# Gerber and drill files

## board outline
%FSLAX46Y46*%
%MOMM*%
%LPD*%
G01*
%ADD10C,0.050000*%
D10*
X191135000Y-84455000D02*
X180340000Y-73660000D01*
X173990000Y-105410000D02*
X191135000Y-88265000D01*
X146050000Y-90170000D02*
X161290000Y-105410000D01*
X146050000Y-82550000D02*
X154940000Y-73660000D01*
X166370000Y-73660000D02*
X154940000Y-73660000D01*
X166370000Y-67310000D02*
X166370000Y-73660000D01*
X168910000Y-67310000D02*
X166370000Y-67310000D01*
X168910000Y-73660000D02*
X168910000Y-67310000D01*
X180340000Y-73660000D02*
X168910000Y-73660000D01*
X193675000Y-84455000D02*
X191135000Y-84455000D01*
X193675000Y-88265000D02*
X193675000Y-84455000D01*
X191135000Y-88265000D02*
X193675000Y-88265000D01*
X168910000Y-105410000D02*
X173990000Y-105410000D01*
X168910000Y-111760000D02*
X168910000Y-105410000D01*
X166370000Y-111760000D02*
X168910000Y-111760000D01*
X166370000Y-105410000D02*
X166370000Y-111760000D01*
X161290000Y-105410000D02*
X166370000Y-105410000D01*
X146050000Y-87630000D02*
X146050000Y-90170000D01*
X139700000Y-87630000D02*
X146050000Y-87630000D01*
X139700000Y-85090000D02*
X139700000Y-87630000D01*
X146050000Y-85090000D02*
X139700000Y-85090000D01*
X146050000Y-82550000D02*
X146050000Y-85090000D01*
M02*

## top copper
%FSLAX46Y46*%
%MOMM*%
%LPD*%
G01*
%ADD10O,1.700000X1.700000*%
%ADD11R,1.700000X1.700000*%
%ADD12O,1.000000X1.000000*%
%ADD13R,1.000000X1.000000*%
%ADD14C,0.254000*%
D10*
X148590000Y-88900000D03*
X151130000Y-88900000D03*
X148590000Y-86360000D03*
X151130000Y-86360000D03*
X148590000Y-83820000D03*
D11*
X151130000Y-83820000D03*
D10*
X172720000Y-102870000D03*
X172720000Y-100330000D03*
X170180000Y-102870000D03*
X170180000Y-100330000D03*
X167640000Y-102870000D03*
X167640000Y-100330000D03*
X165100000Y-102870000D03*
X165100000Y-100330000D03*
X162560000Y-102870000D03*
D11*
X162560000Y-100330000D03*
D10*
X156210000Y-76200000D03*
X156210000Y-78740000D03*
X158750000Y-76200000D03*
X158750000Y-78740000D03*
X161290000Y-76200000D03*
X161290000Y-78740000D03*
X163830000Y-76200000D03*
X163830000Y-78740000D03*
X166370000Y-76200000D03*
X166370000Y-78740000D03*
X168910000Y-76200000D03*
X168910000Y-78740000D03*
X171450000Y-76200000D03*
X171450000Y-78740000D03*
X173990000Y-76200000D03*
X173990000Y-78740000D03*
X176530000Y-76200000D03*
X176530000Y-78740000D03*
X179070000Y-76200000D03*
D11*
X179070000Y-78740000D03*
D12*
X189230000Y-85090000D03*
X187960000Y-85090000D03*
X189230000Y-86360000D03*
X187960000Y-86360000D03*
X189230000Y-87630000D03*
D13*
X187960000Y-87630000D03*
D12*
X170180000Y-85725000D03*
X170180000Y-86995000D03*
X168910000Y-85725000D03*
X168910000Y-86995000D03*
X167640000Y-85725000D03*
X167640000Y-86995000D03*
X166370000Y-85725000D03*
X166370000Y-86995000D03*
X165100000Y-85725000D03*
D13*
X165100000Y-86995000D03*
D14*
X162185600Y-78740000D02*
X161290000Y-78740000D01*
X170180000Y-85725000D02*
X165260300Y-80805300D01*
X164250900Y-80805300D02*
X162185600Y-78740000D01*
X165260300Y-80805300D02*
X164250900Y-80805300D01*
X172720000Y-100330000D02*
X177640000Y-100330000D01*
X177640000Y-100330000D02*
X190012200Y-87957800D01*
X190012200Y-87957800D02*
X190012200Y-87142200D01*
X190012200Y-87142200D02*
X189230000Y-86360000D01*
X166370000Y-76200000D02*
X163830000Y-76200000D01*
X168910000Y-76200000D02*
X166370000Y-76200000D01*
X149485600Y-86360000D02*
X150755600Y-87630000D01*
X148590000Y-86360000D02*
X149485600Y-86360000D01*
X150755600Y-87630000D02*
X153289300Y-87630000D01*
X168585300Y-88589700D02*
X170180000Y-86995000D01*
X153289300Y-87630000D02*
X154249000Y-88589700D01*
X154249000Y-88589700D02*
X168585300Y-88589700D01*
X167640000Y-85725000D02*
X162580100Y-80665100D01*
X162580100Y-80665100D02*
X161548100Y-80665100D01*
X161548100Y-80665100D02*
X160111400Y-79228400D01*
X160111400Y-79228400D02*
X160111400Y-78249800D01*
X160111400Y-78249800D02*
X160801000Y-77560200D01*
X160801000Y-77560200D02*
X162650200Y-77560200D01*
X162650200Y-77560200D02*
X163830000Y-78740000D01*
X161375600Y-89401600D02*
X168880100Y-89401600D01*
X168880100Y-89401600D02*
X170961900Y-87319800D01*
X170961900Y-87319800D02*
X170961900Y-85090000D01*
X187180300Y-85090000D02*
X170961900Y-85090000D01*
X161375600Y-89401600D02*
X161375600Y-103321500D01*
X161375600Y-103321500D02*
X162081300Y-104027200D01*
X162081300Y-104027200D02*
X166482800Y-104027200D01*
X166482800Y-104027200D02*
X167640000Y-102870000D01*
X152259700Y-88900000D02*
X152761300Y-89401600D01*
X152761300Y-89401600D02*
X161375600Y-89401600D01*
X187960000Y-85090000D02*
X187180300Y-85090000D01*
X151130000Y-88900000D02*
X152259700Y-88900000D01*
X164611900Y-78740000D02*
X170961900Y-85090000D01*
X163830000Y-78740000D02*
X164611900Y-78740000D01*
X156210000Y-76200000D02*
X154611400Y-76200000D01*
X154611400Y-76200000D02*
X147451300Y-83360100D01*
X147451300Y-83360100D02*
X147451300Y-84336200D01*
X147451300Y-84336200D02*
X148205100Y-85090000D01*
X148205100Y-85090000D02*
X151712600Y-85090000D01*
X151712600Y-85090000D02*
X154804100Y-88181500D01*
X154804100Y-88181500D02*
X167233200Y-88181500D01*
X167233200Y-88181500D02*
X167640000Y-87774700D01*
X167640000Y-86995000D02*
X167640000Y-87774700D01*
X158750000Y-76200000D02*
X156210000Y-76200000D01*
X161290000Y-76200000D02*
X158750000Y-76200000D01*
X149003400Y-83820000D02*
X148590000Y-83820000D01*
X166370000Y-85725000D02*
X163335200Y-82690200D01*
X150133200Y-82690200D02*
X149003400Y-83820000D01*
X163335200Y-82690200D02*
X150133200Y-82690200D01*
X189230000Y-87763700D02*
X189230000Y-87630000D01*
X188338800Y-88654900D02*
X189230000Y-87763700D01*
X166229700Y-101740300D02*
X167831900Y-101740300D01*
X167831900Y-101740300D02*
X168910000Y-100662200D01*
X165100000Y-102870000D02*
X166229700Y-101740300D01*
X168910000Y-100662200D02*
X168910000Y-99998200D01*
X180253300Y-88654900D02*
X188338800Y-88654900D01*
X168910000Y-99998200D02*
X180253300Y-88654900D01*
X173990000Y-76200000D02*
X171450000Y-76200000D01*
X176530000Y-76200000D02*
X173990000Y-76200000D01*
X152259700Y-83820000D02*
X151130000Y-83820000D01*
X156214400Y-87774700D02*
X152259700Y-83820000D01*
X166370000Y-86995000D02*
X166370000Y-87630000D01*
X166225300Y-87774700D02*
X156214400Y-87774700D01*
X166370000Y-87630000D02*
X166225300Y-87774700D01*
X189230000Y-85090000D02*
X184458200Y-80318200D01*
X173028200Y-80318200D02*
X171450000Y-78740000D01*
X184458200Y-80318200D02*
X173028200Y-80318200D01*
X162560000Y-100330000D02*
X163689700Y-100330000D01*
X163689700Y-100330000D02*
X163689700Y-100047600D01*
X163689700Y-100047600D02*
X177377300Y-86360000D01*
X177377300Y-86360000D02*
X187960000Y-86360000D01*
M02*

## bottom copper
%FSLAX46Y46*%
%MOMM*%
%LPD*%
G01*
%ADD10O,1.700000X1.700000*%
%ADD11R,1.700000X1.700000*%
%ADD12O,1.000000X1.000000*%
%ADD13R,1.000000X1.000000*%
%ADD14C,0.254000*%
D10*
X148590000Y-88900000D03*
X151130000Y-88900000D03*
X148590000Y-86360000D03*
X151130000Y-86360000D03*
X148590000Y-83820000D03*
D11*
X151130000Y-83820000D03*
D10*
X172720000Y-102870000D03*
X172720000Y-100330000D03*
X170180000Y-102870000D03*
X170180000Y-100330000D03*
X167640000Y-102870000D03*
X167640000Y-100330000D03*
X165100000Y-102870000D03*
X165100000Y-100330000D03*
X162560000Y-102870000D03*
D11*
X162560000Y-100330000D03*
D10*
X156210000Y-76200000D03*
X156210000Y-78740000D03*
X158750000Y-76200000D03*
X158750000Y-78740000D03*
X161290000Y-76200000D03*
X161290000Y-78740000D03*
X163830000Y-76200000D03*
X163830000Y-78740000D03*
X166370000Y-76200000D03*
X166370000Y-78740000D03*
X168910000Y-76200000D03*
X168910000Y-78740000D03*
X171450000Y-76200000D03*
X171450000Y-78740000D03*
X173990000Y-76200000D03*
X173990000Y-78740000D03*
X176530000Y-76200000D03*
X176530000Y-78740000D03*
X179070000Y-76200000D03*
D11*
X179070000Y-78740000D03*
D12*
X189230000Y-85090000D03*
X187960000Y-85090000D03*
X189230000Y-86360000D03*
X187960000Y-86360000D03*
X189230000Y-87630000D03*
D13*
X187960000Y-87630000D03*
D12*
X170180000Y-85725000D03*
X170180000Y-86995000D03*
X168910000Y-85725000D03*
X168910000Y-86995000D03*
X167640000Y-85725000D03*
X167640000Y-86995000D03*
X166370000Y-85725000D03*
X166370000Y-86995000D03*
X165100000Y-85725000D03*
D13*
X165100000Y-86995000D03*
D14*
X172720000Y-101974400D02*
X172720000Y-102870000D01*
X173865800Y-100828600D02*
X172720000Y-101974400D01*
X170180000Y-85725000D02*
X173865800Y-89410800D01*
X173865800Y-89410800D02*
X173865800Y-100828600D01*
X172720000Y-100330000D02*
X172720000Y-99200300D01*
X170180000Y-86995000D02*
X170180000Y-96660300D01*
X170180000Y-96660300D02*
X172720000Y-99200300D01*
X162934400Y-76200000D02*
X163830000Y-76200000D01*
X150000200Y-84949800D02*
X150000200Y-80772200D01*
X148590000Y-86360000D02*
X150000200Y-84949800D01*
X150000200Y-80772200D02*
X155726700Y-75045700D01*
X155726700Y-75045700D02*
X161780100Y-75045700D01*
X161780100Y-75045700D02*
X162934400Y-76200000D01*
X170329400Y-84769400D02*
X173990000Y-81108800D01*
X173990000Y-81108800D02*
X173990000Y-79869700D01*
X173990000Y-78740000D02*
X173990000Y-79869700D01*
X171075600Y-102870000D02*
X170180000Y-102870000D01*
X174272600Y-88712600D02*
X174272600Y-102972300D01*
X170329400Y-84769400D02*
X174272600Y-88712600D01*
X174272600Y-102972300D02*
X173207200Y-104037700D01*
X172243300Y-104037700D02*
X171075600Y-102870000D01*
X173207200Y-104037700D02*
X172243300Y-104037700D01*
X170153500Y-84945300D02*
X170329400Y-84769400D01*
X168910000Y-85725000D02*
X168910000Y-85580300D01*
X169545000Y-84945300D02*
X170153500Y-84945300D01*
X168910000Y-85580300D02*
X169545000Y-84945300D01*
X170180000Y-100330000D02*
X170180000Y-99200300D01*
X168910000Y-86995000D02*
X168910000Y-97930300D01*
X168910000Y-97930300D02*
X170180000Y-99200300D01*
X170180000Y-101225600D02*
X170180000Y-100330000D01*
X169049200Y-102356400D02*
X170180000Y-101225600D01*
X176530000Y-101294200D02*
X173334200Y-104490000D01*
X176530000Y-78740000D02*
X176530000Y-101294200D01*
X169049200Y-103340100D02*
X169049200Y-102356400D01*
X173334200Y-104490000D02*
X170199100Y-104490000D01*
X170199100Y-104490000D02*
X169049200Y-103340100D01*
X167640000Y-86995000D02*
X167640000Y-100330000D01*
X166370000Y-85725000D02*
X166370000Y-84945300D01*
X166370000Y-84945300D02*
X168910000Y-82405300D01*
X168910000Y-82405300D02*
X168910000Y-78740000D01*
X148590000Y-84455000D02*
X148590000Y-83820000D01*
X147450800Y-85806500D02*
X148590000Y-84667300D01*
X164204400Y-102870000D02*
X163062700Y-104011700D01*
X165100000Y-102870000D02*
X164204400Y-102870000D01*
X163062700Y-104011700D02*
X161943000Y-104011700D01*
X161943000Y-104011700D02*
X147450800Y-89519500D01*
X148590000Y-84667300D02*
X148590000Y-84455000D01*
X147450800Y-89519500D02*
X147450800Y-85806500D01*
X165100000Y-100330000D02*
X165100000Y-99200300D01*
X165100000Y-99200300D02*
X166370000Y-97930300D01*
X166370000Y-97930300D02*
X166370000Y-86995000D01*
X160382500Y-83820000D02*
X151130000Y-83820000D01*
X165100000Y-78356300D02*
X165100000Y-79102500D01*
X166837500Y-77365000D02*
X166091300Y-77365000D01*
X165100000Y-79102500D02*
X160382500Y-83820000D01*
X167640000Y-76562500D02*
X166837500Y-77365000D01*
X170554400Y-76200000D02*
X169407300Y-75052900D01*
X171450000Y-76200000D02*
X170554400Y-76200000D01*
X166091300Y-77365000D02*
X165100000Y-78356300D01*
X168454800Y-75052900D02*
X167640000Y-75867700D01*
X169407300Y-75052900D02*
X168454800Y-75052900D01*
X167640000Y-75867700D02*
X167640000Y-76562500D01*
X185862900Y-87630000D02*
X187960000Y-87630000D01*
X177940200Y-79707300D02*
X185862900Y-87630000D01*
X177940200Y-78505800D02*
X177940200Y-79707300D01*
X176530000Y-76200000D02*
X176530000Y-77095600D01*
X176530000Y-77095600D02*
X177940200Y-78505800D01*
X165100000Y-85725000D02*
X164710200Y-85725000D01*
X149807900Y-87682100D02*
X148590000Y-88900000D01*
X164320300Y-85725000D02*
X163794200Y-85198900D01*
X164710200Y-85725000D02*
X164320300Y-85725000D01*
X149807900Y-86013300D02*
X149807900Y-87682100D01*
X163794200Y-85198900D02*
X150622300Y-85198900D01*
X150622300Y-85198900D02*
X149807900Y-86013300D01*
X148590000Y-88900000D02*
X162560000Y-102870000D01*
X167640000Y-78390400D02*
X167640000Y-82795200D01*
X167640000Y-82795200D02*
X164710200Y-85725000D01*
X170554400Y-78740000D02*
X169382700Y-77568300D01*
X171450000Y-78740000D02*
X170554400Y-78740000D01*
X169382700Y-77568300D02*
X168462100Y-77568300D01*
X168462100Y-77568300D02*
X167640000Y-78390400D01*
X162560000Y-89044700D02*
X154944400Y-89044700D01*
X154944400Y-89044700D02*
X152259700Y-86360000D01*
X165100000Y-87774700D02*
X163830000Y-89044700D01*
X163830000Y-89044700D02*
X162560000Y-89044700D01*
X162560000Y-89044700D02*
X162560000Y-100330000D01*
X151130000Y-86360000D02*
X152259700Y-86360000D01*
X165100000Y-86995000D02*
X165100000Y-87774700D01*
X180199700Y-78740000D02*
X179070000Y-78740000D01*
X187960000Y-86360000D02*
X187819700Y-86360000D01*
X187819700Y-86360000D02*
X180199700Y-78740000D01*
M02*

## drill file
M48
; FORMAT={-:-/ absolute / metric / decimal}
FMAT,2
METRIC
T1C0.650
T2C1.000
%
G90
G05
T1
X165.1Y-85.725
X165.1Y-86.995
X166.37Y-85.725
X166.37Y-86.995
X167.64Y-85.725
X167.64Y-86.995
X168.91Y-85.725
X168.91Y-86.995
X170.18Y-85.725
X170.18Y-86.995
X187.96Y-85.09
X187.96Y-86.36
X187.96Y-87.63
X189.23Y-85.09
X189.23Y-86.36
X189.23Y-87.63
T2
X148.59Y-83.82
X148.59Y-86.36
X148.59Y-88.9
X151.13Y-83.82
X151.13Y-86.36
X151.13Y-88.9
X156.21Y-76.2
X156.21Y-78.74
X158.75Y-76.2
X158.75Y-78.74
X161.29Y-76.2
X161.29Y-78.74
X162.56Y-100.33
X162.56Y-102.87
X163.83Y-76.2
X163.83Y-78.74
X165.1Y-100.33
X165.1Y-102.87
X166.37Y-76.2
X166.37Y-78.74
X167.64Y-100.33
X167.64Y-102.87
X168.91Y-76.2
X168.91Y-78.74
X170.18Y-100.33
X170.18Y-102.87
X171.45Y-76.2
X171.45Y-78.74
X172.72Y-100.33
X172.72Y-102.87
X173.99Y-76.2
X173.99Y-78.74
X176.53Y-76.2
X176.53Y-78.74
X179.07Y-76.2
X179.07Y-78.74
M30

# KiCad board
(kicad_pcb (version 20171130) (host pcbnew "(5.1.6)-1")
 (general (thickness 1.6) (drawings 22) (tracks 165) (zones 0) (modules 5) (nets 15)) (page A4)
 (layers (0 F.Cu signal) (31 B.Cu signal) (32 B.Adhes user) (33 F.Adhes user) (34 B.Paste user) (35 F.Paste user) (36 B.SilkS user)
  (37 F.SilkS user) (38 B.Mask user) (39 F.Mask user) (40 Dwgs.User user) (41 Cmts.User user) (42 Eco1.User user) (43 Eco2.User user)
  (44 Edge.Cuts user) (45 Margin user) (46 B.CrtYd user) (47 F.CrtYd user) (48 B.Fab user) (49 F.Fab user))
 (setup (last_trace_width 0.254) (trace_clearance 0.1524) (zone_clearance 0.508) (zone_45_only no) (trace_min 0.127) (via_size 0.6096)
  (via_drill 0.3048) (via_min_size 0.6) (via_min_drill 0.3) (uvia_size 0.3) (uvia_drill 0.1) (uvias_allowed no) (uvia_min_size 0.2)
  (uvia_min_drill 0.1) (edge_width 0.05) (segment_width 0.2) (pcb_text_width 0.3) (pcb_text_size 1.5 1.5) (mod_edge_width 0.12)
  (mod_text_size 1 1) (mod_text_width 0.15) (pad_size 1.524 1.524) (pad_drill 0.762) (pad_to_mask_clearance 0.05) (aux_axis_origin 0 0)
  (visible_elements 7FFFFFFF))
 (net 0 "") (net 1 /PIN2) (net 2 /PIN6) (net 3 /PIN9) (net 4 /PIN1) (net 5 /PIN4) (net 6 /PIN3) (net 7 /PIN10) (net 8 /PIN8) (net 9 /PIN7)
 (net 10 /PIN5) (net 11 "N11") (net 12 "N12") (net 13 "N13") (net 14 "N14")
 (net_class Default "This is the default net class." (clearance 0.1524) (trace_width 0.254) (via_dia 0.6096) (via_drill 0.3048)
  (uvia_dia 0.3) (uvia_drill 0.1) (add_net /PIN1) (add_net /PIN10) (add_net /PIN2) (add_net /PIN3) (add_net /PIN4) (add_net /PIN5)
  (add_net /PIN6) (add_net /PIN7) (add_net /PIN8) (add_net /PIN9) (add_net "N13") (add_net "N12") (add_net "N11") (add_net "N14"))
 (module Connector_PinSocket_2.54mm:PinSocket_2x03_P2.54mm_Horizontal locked (layer F.Cu) (at 151.13 83.82)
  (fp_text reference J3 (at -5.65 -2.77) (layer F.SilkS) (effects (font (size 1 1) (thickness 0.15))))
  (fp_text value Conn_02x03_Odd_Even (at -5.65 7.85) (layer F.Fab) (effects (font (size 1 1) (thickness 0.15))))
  (pad 6 thru_hole oval (at -2.54 5.08) (size 1.7 1.7) (drill 1) (layers *.Cu *.Mask) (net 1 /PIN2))
  (pad 5 thru_hole oval (at 0 5.08) (size 1.7 1.7) (drill 1) (layers *.Cu *.Mask) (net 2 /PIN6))
  (pad 4 thru_hole oval (at -2.54 2.54) (size 1.7 1.7) (drill 1) (layers *.Cu *.Mask) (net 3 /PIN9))
  (pad 3 thru_hole oval (at 0 2.54) (size 1.7 1.7) (drill 1) (layers *.Cu *.Mask) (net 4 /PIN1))
  (pad 2 thru_hole oval (at -2.54 0) (size 1.7 1.7) (drill 1) (layers *.Cu *.Mask) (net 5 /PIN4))
  (pad 1 thru_hole rect (at 0 0) (size 1.7 1.7) (drill 1) (layers *.Cu *.Mask) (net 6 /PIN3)))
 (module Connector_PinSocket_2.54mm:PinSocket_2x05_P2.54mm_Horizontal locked (layer F.Cu) (at 162.56 100.33 90)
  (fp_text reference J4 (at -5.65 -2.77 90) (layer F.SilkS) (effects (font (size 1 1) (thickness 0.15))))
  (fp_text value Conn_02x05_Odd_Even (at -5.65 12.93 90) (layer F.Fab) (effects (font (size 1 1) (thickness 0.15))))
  (pad 10 thru_hole oval (at -2.54 10.16 90) (size 1.7 1.7) (drill 1) (layers *.Cu *.Mask) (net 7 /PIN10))
  (pad 9 thru_hole oval (at 0 10.16 90) (size 1.7 1.7) (drill 1) (layers *.Cu *.Mask) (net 3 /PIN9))
  (pad 8 thru_hole oval (at -2.54 7.62 90) (size 1.7 1.7) (drill 1) (layers *.Cu *.Mask) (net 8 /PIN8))
  (pad 7 thru_hole oval (at 0 7.62 90) (size 1.7 1.7) (drill 1) (layers *.Cu *.Mask) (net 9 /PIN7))
  (pad 6 thru_hole oval (at -2.54 5.08 90) (size 1.7 1.7) (drill 1) (layers *.Cu *.Mask) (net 2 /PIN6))
  (pad 5 thru_hole oval (at 0 5.08 90) (size 1.7 1.7) (drill 1) (layers *.Cu *.Mask) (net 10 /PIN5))
  (pad 4 thru_hole oval (at -2.54 2.54 90) (size 1.7 1.7) (drill 1) (layers *.Cu *.Mask) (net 5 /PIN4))
  (pad 3 thru_hole oval (at 0 2.54 90) (size 1.7 1.7) (drill 1) (layers *.Cu *.Mask) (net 6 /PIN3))
  (pad 2 thru_hole oval (at -2.54 0 90) (size 1.7 1.7) (drill 1) (layers *.Cu *.Mask) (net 1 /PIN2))
  (pad 1 thru_hole rect (at 0 0 90) (size 1.7 1.7) (drill 1) (layers *.Cu *.Mask) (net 4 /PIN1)))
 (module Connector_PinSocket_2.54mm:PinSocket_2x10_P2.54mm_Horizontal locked (layer F.Cu) (at 179.07 78.74 270)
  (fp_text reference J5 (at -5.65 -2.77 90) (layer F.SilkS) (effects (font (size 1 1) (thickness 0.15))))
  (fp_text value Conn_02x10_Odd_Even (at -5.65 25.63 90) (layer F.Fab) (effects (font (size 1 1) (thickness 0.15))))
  (pad 20 thru_hole oval (at -2.54 22.86 270) (size 1.7 1.7) (drill 1) (layers *.Cu *.Mask) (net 10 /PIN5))
  (pad 19 thru_hole oval (at 0 22.86 270) (size 1.7 1.7) (drill 1) (layers *.Cu *.Mask) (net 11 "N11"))
  (pad 18 thru_hole oval (at -2.54 20.32 270) (size 1.7 1.7) (drill 1) (layers *.Cu *.Mask) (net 10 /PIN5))
  (pad 17 thru_hole oval (at 0 20.32 270) (size 1.7 1.7) (drill 1) (layers *.Cu *.Mask) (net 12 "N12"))
  (pad 16 thru_hole oval (at -2.54 17.78 270) (size 1.7 1.7) (drill 1) (layers *.Cu *.Mask) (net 10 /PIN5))
  (pad 15 thru_hole oval (at 0 17.78 270) (size 1.7 1.7) (drill 1) (layers *.Cu *.Mask) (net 7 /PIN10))
  (pad 14 thru_hole oval (at -2.54 15.24 270) (size 1.7 1.7) (drill 1) (layers *.Cu *.Mask) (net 3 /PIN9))
  (pad 13 thru_hole oval (at 0 15.24 270) (size 1.7 1.7) (drill 1) (layers *.Cu *.Mask) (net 2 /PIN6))
  (pad 12 thru_hole oval (at -2.54 12.7 270) (size 1.7 1.7) (drill 1) (layers *.Cu *.Mask) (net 3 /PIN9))
  (pad 11 thru_hole oval (at 0 12.7 270) (size 1.7 1.7) (drill 1) (layers *.Cu *.Mask) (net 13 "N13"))
  (pad 10 thru_hole oval (at -2.54 10.16 270) (size 1.7 1.7) (drill 1) (layers *.Cu *.Mask) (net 3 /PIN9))
  (pad 9 thru_hole oval (at 0 10.16 270) (size 1.7 1.7) (drill 1) (layers *.Cu *.Mask) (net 5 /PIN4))
  (pad 8 thru_hole oval (at -2.54 7.62 270) (size 1.7 1.7) (drill 1) (layers *.Cu *.Mask) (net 6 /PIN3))
  (pad 7 thru_hole oval (at 0 7.62 270) (size 1.7 1.7) (drill 1) (layers *.Cu *.Mask) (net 1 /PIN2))
  (pad 6 thru_hole oval (at -2.54 5.08 270) (size 1.7 1.7) (drill 1) (layers *.Cu *.Mask) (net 6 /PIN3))
  (pad 5 thru_hole oval (at 0 5.08 270) (size 1.7 1.7) (drill 1) (layers *.Cu *.Mask) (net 8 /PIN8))
  (pad 4 thru_hole oval (at -2.54 2.54 270) (size 1.7 1.7) (drill 1) (layers *.Cu *.Mask) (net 6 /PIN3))
  (pad 3 thru_hole oval (at 0 2.54 270) (size 1.7 1.7) (drill 1) (layers *.Cu *.Mask) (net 9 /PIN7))
  (pad 2 thru_hole oval (at -2.54 0 270) (size 1.7 1.7) (drill 1) (layers *.Cu *.Mask) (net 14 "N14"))
  (pad 1 thru_hole rect (at 0 0 270) (size 1.7 1.7) (drill 1) (layers *.Cu *.Mask) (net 4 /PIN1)))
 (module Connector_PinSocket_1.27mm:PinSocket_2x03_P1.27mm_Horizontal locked (layer F.Cu) (at 187.96 87.63 180)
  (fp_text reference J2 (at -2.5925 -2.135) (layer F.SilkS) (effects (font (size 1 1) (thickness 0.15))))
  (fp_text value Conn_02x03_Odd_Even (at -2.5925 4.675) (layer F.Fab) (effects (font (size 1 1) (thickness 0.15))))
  (pad 6 thru_hole oval (at -1.27 2.54 180) (size 1 1) (drill 0.65) (layers *.Cu *.Mask) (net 1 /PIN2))
  (pad 5 thru_hole oval (at 0 2.54 180) (size 1 1) (drill 0.65) (layers *.Cu *.Mask) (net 2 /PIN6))
  (pad 4 thru_hole oval (at -1.27 1.27 180) (size 1 1) (drill 0.65) (layers *.Cu *.Mask) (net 3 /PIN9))
  (pad 3 thru_hole oval (at 0 1.27 180) (size 1 1) (drill 0.65) (layers *.Cu *.Mask) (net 4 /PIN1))
  (pad 2 thru_hole oval (at -1.27 0 180) (size 1 1) (drill 0.65) (layers *.Cu *.Mask) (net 5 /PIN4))
  (pad 1 thru_hole rect (at 0 0 180) (size 1 1) (drill 0.65) (layers *.Cu *.Mask) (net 6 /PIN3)))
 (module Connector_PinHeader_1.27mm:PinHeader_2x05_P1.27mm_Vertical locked (layer F.Cu) (at 165.1 86.995 90)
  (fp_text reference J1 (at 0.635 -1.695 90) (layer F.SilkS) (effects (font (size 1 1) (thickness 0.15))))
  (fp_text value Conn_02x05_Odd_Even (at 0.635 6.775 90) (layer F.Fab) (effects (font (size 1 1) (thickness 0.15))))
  (pad 10 thru_hole oval (at 1.27 5.08 90) (size 1 1) (drill 0.65) (layers *.Cu *.Mask) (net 7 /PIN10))
  (pad 9 thru_hole oval (at 0 5.08 90) (size 1 1) (drill 0.65) (layers *.Cu *.Mask) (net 3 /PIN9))
  (pad 8 thru_hole oval (at 1.27 3.81 90) (size 1 1) (drill 0.65) (layers *.Cu *.Mask) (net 8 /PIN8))
  (pad 7 thru_hole oval (at 0 3.81 90) (size 1 1) (drill 0.65) (layers *.Cu *.Mask) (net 9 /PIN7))
  (pad 6 thru_hole oval (at 1.27 2.54 90) (size 1 1) (drill 0.65) (layers *.Cu *.Mask) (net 2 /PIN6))
  (pad 5 thru_hole oval (at 0 2.54 90) (size 1 1) (drill 0.65) (layers *.Cu *.Mask) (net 10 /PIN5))
  (pad 4 thru_hole oval (at 1.27 1.27 90) (size 1 1) (drill 0.65) (layers *.Cu *.Mask) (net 5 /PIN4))
  (pad 3 thru_hole oval (at 0 1.27 90) (size 1 1) (drill 0.65) (layers *.Cu *.Mask) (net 6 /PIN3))
  (pad 2 thru_hole oval (at 1.27 0 90) (size 1 1) (drill 0.65) (layers *.Cu *.Mask) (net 1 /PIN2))
  (pad 1 thru_hole rect (at 0 0 90) (size 1 1) (drill 0.65) (layers *.Cu *.Mask) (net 4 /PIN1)))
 (gr_line (start 191.135 84.455) (end 180.34 73.66) (layer Edge.Cuts) (width 0.05))
 (gr_line (start 173.99 105.41) (end 191.135 88.265) (layer Edge.Cuts) (width 0.05))
 (gr_line (start 146.05 90.17) (end 161.29 105.41) (layer Edge.Cuts) (width 0.05))
 (gr_line (start 146.05 82.55) (end 154.94 73.66) (layer Edge.Cuts) (width 0.05))
 (gr_line (start 166.37 73.66) (end 154.94 73.66) (layer Edge.Cuts) (width 0.05))
 (gr_line (start 166.37 67.31) (end 166.37 73.66) (layer Edge.Cuts) (width 0.05))
 (gr_line (start 168.91 67.31) (end 166.37 67.31) (layer Edge.Cuts) (width 0.05))
 (gr_line (start 168.91 73.66) (end 168.91 67.31) (layer Edge.Cuts) (width 0.05))
 (gr_line (start 180.34 73.66) (end 168.91 73.66) (layer Edge.Cuts) (width 0.05))
 (gr_line (start 193.675 84.455) (end 191.135 84.455) (layer Edge.Cuts) (width 0.05))
 (gr_line (start 193.675 88.265) (end 193.675 84.455) (layer Edge.Cuts) (width 0.05))
 (gr_line (start 191.135 88.265) (end 193.675 88.265) (layer Edge.Cuts) (width 0.05))
 (gr_line (start 168.91 105.41) (end 173.99 105.41) (layer Edge.Cuts) (width 0.05))
 (gr_line (start 168.91 111.76) (end 168.91 105.41) (layer Edge.Cuts) (width 0.05))
 (gr_line (start 166.37 111.76) (end 168.91 111.76) (layer Edge.Cuts) (width 0.05))
 (gr_line (start 166.37 105.41) (end 166.37 111.76) (layer Edge.Cuts) (width 0.05))
 (gr_line (start 161.29 105.41) (end 166.37 105.41) (layer Edge.Cuts) (width 0.05))
 (gr_line (start 146.05 87.63) (end 146.05 90.17) (layer Edge.Cuts) (width 0.05))
 (gr_line (start 139.7 87.63) (end 146.05 87.63) (layer Edge.Cuts) (width 0.05))
 (gr_line (start 139.7 85.09) (end 139.7 87.63) (layer Edge.Cuts) (width 0.05))
 (gr_line (start 146.05 85.09) (end 139.7 85.09) (layer Edge.Cuts) (width 0.05))
 (gr_line (start 146.05 82.55) (end 146.05 85.09) (layer Edge.Cuts) (width 0.05))
 (segment (start 162.1856 78.74) (end 161.29 78.74) (width 0.254) (layer F.Cu) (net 7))
 (segment (start 170.18 85.725) (end 165.2603 80.8053) (width 0.254) (layer F.Cu) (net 7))
 (segment (start 164.2509 80.8053) (end 162.1856 78.74) (width 0.254) (layer F.Cu) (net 7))
 (segment (start 165.2603 80.8053) (end 164.2509 80.8053) (width 0.254) (layer F.Cu) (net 7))
 (segment (start 172.72 101.9744) (end 172.72 102.87) (width 0.254) (layer B.Cu) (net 7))
 (segment (start 173.8658 100.8286) (end 172.72 101.9744) (width 0.254) (layer B.Cu) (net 7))
 (segment (start 170.18 85.725) (end 173.8658 89.4108) (width 0.254) (layer B.Cu) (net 7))
 (segment (start 173.8658 89.4108) (end 173.8658 100.8286) (width 0.254) (layer B.Cu) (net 7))
 (segment (start 172.72 100.33) (end 172.72 99.2003) (width 0.254) (layer B.Cu) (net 3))
 (segment (start 170.18 86.995) (end 170.18 96.6603) (width 0.254) (layer B.Cu) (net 3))
 (segment (start 170.18 96.6603) (end 172.72 99.2003) (width 0.254) (layer B.Cu) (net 3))
 (segment (start 172.72 100.33) (end 177.64 100.33) (width 0.254) (layer F.Cu) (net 3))
 (segment (start 177.64 100.33) (end 190.0122 87.9578) (width 0.254) (layer F.Cu) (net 3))
 (segment (start 190.0122 87.9578) (end 190.0122 87.1422) (width 0.254) (layer F.Cu) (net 3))
 (segment (start 190.0122 87.1422) (end 189.23 86.36) (width 0.254) (layer F.Cu) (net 3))
 (segment (start 166.37 76.2) (end 163.83 76.2) (width 0.254) (layer F.Cu) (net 3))
 (segment (start 168.91 76.2) (end 166.37 76.2) (width 0.254) (layer F.Cu) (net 3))
 (segment (start 149.4856 86.36) (end 150.7556 87.63) (width 0.254) (layer F.Cu) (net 3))
 (segment (start 148.59 86.36) (end 149.4856 86.36) (width 0.254) (layer F.Cu) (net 3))
 (segment (start 150.7556 87.63) (end 153.2893 87.63) (width 0.254) (layer F.Cu) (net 3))
 (segment (start 168.5853 88.5897) (end 170.18 86.995) (width 0.254) (layer F.Cu) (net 3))
 (segment (start 153.2893 87.63) (end 154.249 88.5897) (width 0.254) (layer F.Cu) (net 3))
 (segment (start 154.249 88.5897) (end 168.5853 88.5897) (width 0.254) (layer F.Cu) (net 3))
 (segment (start 162.9344 76.2) (end 163.83 76.2) (width 0.254) (layer B.Cu) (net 3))
 (segment (start 150.0002 84.9498) (end 150.0002 80.7722) (width 0.254) (layer B.Cu) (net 3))
 (segment (start 148.59 86.36) (end 150.0002 84.9498) (width 0.254) (layer B.Cu) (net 3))
 (segment (start 150.0002 80.7722) (end 155.7267 75.0457) (width 0.254) (layer B.Cu) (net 3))
 (segment (start 155.7267 75.0457) (end 161.7801 75.0457) (width 0.254) (layer B.Cu) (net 3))
 (segment (start 161.7801 75.0457) (end 162.9344 76.2) (width 0.254) (layer B.Cu) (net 3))
 (segment (start 170.3294 84.7694) (end 173.99 81.1088) (width 0.254) (layer B.Cu) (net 8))
 (segment (start 173.99 81.1088) (end 173.99 79.8697) (width 0.254) (layer B.Cu) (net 8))
 (segment (start 173.99 78.74) (end 173.99 79.8697) (width 0.254) (layer B.Cu) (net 8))
 (segment (start 171.0756 102.87) (end 170.18 102.87) (width 0.254) (layer B.Cu) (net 8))
 (segment (start 174.2726 88.7126) (end 174.2726 102.9723) (width 0.254) (layer B.Cu) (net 8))
 (segment (start 170.3294 84.7694) (end 174.2726 88.7126) (width 0.254) (layer B.Cu) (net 8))
 (segment (start 174.2726 102.9723) (end 173.2072 104.0377) (width 0.254) (layer B.Cu) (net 8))
 (segment (start 172.2433 104.0377) (end 171.0756 102.87) (width 0.254) (layer B.Cu) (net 8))
 (segment (start 173.2072 104.0377) (end 172.2433 104.0377) (width 0.254) (layer B.Cu) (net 8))
 (segment (start 170.1535 84.9453) (end 170.3294 84.7694) (width 0.254) (layer B.Cu) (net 8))
 (segment (start 168.91 85.725) (end 168.91 85.5803) (width 0.254) (layer B.Cu) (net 8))
 (segment (start 169.545 84.9453) (end 170.1535 84.9453) (width 0.254) (layer B.Cu) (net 8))
 (segment (start 168.91 85.5803) (end 169.545 84.9453) (width 0.254) (layer B.Cu) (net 8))
 (segment (start 170.18 100.33) (end 170.18 99.2003) (width 0.254) (layer B.Cu) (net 9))
 (segment (start 168.91 86.995) (end 168.91 97.9303) (width 0.254) (layer B.Cu) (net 9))
 (segment (start 168.91 97.9303) (end 170.18 99.2003) (width 0.254) (layer B.Cu) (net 9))
 (segment (start 170.18 101.2256) (end 170.18 100.33) (width 0.254) (layer B.Cu) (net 9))
 (segment (start 169.0492 102.3564) (end 170.18 101.2256) (width 0.254) (layer B.Cu) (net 9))
 (segment (start 176.53 101.2942) (end 173.3342 104.49) (width 0.254) (layer B.Cu) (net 9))
 (segment (start 176.53 78.74) (end 176.53 101.2942) (width 0.254) (layer B.Cu) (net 9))
 (segment (start 169.0492 103.3401) (end 169.0492 102.3564) (width 0.254) (layer B.Cu) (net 9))
 (segment (start 173.3342 104.49) (end 170.1991 104.49) (width 0.254) (layer B.Cu) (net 9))
 (segment (start 170.1991 104.49) (end 169.0492 103.3401) (width 0.254) (layer B.Cu) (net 9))
 (segment (start 167.64 85.725) (end 162.5801 80.6651) (width 0.254) (layer F.Cu) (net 2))
 (segment (start 162.5801 80.6651) (end 161.5481 80.6651) (width 0.254) (layer F.Cu) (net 2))
 (segment (start 161.5481 80.6651) (end 160.1114 79.2284) (width 0.254) (layer F.Cu) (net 2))
 (segment (start 160.1114 79.2284) (end 160.1114 78.2498) (width 0.254) (layer F.Cu) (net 2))
 (segment (start 160.1114 78.2498) (end 160.801 77.5602) (width 0.254) (layer F.Cu) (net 2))
 (segment (start 160.801 77.5602) (end 162.6502 77.5602) (width 0.254) (layer F.Cu) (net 2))
 (segment (start 162.6502 77.5602) (end 163.83 78.74) (width 0.254) (layer F.Cu) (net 2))
 (segment (start 161.3756 89.4016) (end 168.8801 89.4016) (width 0.254) (layer F.Cu) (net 2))
 (segment (start 168.8801 89.4016) (end 170.9619 87.3198) (width 0.254) (layer F.Cu) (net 2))
 (segment (start 170.9619 87.3198) (end 170.9619 85.09) (width 0.254) (layer F.Cu) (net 2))
 (segment (start 187.1803 85.09) (end 170.9619 85.09) (width 0.254) (layer F.Cu) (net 2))
 (segment (start 161.3756 89.4016) (end 161.3756 103.3215) (width 0.254) (layer F.Cu) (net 2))
 (segment (start 161.3756 103.3215) (end 162.0813 104.0272) (width 0.254) (layer F.Cu) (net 2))
 (segment (start 162.0813 104.0272) (end 166.4828 104.0272) (width 0.254) (layer F.Cu) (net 2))
 (segment (start 166.4828 104.0272) (end 167.64 102.87) (width 0.254) (layer F.Cu) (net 2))
 (segment (start 152.2597 88.9) (end 152.7613 89.4016) (width 0.254) (layer F.Cu) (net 2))
 (segment (start 152.7613 89.4016) (end 161.3756 89.4016) (width 0.254) (layer F.Cu) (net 2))
 (segment (start 187.96 85.09) (end 187.1803 85.09) (width 0.254) (layer F.Cu) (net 2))
 (segment (start 151.13 88.9) (end 152.2597 88.9) (width 0.254) (layer F.Cu) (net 2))
 (segment (start 164.6119 78.74) (end 170.9619 85.09) (width 0.254) (layer F.Cu) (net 2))
 (segment (start 163.83 78.74) (end 164.6119 78.74) (width 0.254) (layer F.Cu) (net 2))
 (segment (start 156.21 76.2) (end 154.6114 76.2) (width 0.254) (layer F.Cu) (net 10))
 (segment (start 154.6114 76.2) (end 147.4513 83.3601) (width 0.254) (layer F.Cu) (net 10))
 (segment (start 147.4513 83.3601) (end 147.4513 84.3362) (width 0.254) (layer F.Cu) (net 10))
 (segment (start 147.4513 84.3362) (end 148.2051 85.09) (width 0.254) (layer F.Cu) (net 10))
 (segment (start 148.2051 85.09) (end 151.7126 85.09) (width 0.254) (layer F.Cu) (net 10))
 (segment (start 151.7126 85.09) (end 154.8041 88.1815) (width 0.254) (layer F.Cu) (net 10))
 (segment (start 154.8041 88.1815) (end 167.2332 88.1815) (width 0.254) (layer F.Cu) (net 10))
 (segment (start 167.2332 88.1815) (end 167.64 87.7747) (width 0.254) (layer F.Cu) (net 10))
 (segment (start 167.64 86.995) (end 167.64 87.7747) (width 0.254) (layer F.Cu) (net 10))
 (segment (start 167.64 86.995) (end 167.64 100.33) (width 0.254) (layer B.Cu) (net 10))
 (segment (start 158.75 76.2) (end 156.21 76.2) (width 0.254) (layer F.Cu) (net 10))
 (segment (start 161.29 76.2) (end 158.75 76.2) (width 0.254) (layer F.Cu) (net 10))
 (segment (start 166.37 85.725) (end 166.37 84.9453) (width 0.254) (layer B.Cu) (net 5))
 (segment (start 166.37 84.9453) (end 168.91 82.4053) (width 0.254) (layer B.Cu) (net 5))
 (segment (start 168.91 82.4053) (end 168.91 78.74) (width 0.254) (layer B.Cu) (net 5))
 (segment (start 149.0034 83.82) (end 148.59 83.82) (width 0.254) (layer F.Cu) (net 5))
 (segment (start 166.37 85.725) (end 163.3352 82.6902) (width 0.254) (layer F.Cu) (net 5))
 (segment (start 150.1332 82.6902) (end 149.0034 83.82) (width 0.254) (layer F.Cu) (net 5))
 (segment (start 163.3352 82.6902) (end 150.1332 82.6902) (width 0.254) (layer F.Cu) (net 5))
 (segment (start 148.59 84.455) (end 148.59 83.82) (width 0.254) (layer B.Cu) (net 5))
 (segment (start 147.4508 85.8065) (end 148.59 84.6673) (width 0.254) (layer B.Cu) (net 5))
 (segment (start 164.2044 102.87) (end 163.0627 104.0117) (width 0.254) (layer B.Cu) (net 5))
 (segment (start 165.1 102.87) (end 164.2044 102.87) (width 0.254) (layer B.Cu) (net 5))
 (segment (start 163.0627 104.0117) (end 161.943 104.0117) (width 0.254) (layer B.Cu) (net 5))
 (segment (start 161.943 104.0117) (end 147.4508 89.5195) (width 0.254) (layer B.Cu) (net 5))
 (segment (start 148.59 84.6673) (end 148.59 84.455) (width 0.254) (layer B.Cu) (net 5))
 (segment (start 147.4508 89.5195) (end 147.4508 85.8065) (width 0.254) (layer B.Cu) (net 5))
 (segment (start 189.23 87.7637) (end 189.23 87.63) (width 0.254) (layer F.Cu) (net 5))
 (segment (start 188.3388 88.6549) (end 189.23 87.7637) (width 0.254) (layer F.Cu) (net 5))
 (segment (start 166.2297 101.7403) (end 167.8319 101.7403) (width 0.254) (layer F.Cu) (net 5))
 (segment (start 167.8319 101.7403) (end 168.91 100.6622) (width 0.254) (layer F.Cu) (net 5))
 (segment (start 165.1 102.87) (end 166.2297 101.7403) (width 0.254) (layer F.Cu) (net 5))
 (segment (start 168.91 100.6622) (end 168.91 99.9982) (width 0.254) (layer F.Cu) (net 5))
 (segment (start 180.2533 88.6549) (end 188.3388 88.6549) (width 0.254) (layer F.Cu) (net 5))
 (segment (start 168.91 99.9982) (end 180.2533 88.6549) (width 0.254) (layer F.Cu) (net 5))
 (segment (start 173.99 76.2) (end 171.45 76.2) (width 0.254) (layer F.Cu) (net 6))
 (segment (start 165.1 100.33) (end 165.1 99.2003) (width 0.254) (layer B.Cu) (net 6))
 (segment (start 165.1 99.2003) (end 166.37 97.9303) (width 0.254) (layer B.Cu) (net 6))
 (segment (start 166.37 97.9303) (end 166.37 86.995) (width 0.254) (layer B.Cu) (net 6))
 (segment (start 176.53 76.2) (end 173.99 76.2) (width 0.254) (layer F.Cu) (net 6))
 (segment (start 160.3825 83.82) (end 151.13 83.82) (width 0.254) (layer B.Cu) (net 6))
 (segment (start 165.1 78.3563) (end 165.1 79.1025) (width 0.254) (layer B.Cu) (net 6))
 (segment (start 166.8375 77.365) (end 166.0913 77.365) (width 0.254) (layer B.Cu) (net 6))
 (segment (start 165.1 79.1025) (end 160.3825 83.82) (width 0.254) (layer B.Cu) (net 6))
 (segment (start 167.64 76.5625) (end 166.8375 77.365) (width 0.254) (layer B.Cu) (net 6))
 (segment (start 170.5544 76.2) (end 169.4073 75.0529) (width 0.254) (layer B.Cu) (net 6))
 (segment (start 171.45 76.2) (end 170.5544 76.2) (width 0.254) (layer B.Cu) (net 6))
 (segment (start 166.0913 77.365) (end 165.1 78.3563) (width 0.254) (layer B.Cu) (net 6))
 (segment (start 168.4548 75.0529) (end 167.64 75.8677) (width 0.254) (layer B.Cu) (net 6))
 (segment (start 169.4073 75.0529) (end 168.4548 75.0529) (width 0.254) (layer B.Cu) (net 6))
 (segment (start 167.64 75.8677) (end 167.64 76.5625) (width 0.254) (layer B.Cu) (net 6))
 (segment (start 185.8629 87.63) (end 187.96 87.63) (width 0.254) (layer B.Cu) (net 6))
 (segment (start 177.9402 79.7073) (end 185.8629 87.63) (width 0.254) (layer B.Cu) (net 6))
 (segment (start 177.9402 78.5058) (end 177.9402 79.7073) (width 0.254) (layer B.Cu) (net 6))
 (segment (start 176.53 76.2) (end 176.53 77.0956) (width 0.254) (layer B.Cu) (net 6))
 (segment (start 176.53 77.0956) (end 177.9402 78.5058) (width 0.254) (layer B.Cu) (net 6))
 (segment (start 152.2597 83.82) (end 151.13 83.82) (width 0.254) (layer F.Cu) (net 6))
 (segment (start 156.2144 87.7747) (end 152.2597 83.82) (width 0.254) (layer F.Cu) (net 6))
 (segment (start 166.37 86.995) (end 166.37 87.63) (width 0.254) (layer F.Cu) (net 6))
 (segment (start 166.2253 87.7747) (end 156.2144 87.7747) (width 0.254) (layer F.Cu) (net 6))
 (segment (start 166.37 87.63) (end 166.2253 87.7747) (width 0.254) (layer F.Cu) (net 6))
 (segment (start 165.1 85.725) (end 164.7102 85.725) (width 0.254) (layer B.Cu) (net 1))
 (segment (start 149.8079 87.6821) (end 148.59 88.9) (width 0.254) (layer B.Cu) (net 1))
 (segment (start 164.3203 85.725) (end 163.7942 85.1989) (width 0.254) (layer B.Cu) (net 1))
 (segment (start 164.7102 85.725) (end 164.3203 85.725) (width 0.254) (layer B.Cu) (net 1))
 (segment (start 149.8079 86.0133) (end 149.8079 87.6821) (width 0.254) (layer B.Cu) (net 1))
 (segment (start 163.7942 85.1989) (end 150.6223 85.1989) (width 0.254) (layer B.Cu) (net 1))
 (segment (start 150.6223 85.1989) (end 149.8079 86.0133) (width 0.254) (layer B.Cu) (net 1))
 (segment (start 148.59 88.9) (end 162.56 102.87) (width 0.254) (layer B.Cu) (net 1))
 (segment (start 167.64 78.3904) (end 167.64 82.7952) (width 0.254) (layer B.Cu) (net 1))
 (segment (start 167.64 82.7952) (end 164.7102 85.725) (width 0.254) (layer B.Cu) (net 1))
 (segment (start 170.5544 78.74) (end 169.3827 77.5683) (width 0.254) (layer B.Cu) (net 1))
 (segment (start 171.45 78.74) (end 170.5544 78.74) (width 0.254) (layer B.Cu) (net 1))
 (segment (start 169.3827 77.5683) (end 168.4621 77.5683) (width 0.254) (layer B.Cu) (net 1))
 (segment (start 168.4621 77.5683) (end 167.64 78.3904) (width 0.254) (layer B.Cu) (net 1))
 (segment (start 189.23 85.09) (end 184.4582 80.3182) (width 0.254) (layer F.Cu) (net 1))
 (segment (start 173.0282 80.3182) (end 171.45 78.74) (width 0.254) (layer F.Cu) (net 1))
 (segment (start 184.4582 80.3182) (end 173.0282 80.3182) (width 0.254) (layer F.Cu) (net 1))
 (segment (start 162.56 89.0447) (end 154.9444 89.0447) (width 0.254) (layer B.Cu) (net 4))
 (segment (start 154.9444 89.0447) (end 152.2597 86.36) (width 0.254) (layer B.Cu) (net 4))
 (segment (start 165.1 87.7747) (end 163.83 89.0447) (width 0.254) (layer B.Cu) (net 4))
 (segment (start 163.83 89.0447) (end 162.56 89.0447) (width 0.254) (layer B.Cu) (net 4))
 (segment (start 162.56 89.0447) (end 162.56 100.33) (width 0.254) (layer B.Cu) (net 4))
 (segment (start 151.13 86.36) (end 152.2597 86.36) (width 0.254) (layer B.Cu) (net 4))
 (segment (start 165.1 86.995) (end 165.1 87.7747) (width 0.254) (layer B.Cu) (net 4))
 (segment (start 162.56 100.33) (end 163.6897 100.33) (width 0.254) (layer F.Cu) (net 4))
 (segment (start 163.6897 100.33) (end 163.6897 100.0476) (width 0.254) (layer F.Cu) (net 4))
 (segment (start 163.6897 100.0476) (end 177.3773 86.36) (width 0.254) (layer F.Cu) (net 4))
 (segment (start 177.3773 86.36) (end 187.96 86.36) (width 0.254) (layer F.Cu) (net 4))
 (segment (start 180.1997 78.74) (end 179.07 78.74) (width 0.254) (layer B.Cu) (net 4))
 (segment (start 187.96 86.36) (end 187.8197 86.36) (width 0.254) (layer B.Cu) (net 4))
 (segment (start 187.8197 86.36) (end 180.1997 78.74) (width 0.254) (layer B.Cu) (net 4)))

